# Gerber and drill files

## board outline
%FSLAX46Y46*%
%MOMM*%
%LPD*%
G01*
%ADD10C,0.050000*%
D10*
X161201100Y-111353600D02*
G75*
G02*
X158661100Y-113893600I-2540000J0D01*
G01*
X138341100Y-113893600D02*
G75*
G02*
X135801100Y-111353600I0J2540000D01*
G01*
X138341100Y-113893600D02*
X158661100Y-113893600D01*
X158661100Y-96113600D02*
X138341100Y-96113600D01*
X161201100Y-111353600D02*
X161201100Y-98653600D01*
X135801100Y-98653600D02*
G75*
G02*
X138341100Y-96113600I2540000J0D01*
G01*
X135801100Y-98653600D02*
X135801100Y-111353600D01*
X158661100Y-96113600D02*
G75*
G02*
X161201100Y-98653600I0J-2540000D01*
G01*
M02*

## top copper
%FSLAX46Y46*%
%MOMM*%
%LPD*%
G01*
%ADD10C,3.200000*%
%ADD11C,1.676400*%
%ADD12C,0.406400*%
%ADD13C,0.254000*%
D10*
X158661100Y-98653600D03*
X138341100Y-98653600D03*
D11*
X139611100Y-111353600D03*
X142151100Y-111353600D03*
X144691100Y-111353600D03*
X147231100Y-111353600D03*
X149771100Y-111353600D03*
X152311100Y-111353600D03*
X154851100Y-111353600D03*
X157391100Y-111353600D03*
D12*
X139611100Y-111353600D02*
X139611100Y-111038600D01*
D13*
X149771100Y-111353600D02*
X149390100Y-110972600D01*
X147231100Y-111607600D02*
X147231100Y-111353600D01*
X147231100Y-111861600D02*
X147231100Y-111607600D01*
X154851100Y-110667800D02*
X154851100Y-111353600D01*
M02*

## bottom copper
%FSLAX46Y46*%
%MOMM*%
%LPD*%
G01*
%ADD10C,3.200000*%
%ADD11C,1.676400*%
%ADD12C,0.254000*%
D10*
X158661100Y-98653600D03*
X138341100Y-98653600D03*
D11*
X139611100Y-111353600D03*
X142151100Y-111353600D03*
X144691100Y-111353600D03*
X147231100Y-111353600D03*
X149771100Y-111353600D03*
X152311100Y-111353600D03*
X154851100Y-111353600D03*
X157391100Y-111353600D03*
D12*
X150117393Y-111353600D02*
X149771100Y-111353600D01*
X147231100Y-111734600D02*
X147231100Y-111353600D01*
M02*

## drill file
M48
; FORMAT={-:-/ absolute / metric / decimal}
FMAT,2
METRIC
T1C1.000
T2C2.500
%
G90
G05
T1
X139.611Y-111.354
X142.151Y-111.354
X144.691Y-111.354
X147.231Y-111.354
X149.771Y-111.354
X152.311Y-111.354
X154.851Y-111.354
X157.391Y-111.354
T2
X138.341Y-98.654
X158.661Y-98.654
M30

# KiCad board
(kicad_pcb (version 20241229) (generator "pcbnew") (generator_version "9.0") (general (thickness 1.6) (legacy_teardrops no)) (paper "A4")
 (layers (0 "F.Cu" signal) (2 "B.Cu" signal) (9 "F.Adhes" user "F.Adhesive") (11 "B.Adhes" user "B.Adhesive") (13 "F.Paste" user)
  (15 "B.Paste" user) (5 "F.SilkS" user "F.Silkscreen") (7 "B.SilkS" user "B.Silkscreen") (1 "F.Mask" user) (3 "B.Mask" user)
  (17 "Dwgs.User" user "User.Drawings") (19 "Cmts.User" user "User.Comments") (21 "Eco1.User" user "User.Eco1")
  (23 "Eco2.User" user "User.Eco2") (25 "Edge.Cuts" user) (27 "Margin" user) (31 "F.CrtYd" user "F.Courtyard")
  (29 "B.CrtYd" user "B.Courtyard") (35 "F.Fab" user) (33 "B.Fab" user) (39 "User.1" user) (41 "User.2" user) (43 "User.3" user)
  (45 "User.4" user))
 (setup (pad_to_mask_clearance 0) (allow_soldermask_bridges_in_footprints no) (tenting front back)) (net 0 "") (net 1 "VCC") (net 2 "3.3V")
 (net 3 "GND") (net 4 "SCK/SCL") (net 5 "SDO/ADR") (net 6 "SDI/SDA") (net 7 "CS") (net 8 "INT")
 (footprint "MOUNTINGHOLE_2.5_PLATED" (layer "F.Cu") (at 158.6611 98.6536)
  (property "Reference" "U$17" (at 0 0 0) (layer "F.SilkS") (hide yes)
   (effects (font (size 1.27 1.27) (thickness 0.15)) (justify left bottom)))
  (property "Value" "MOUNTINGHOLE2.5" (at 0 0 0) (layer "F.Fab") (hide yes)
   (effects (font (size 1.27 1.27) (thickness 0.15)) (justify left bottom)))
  (pad "P$1" thru_hole circle (at 0 0) (size 3.2 3.2) (drill 2.5) (layers "*.Cu" "*.Mask") (remove_unused_layers no)
   (solder_mask_margin 0.0508) (thermal_bridge_angle 0))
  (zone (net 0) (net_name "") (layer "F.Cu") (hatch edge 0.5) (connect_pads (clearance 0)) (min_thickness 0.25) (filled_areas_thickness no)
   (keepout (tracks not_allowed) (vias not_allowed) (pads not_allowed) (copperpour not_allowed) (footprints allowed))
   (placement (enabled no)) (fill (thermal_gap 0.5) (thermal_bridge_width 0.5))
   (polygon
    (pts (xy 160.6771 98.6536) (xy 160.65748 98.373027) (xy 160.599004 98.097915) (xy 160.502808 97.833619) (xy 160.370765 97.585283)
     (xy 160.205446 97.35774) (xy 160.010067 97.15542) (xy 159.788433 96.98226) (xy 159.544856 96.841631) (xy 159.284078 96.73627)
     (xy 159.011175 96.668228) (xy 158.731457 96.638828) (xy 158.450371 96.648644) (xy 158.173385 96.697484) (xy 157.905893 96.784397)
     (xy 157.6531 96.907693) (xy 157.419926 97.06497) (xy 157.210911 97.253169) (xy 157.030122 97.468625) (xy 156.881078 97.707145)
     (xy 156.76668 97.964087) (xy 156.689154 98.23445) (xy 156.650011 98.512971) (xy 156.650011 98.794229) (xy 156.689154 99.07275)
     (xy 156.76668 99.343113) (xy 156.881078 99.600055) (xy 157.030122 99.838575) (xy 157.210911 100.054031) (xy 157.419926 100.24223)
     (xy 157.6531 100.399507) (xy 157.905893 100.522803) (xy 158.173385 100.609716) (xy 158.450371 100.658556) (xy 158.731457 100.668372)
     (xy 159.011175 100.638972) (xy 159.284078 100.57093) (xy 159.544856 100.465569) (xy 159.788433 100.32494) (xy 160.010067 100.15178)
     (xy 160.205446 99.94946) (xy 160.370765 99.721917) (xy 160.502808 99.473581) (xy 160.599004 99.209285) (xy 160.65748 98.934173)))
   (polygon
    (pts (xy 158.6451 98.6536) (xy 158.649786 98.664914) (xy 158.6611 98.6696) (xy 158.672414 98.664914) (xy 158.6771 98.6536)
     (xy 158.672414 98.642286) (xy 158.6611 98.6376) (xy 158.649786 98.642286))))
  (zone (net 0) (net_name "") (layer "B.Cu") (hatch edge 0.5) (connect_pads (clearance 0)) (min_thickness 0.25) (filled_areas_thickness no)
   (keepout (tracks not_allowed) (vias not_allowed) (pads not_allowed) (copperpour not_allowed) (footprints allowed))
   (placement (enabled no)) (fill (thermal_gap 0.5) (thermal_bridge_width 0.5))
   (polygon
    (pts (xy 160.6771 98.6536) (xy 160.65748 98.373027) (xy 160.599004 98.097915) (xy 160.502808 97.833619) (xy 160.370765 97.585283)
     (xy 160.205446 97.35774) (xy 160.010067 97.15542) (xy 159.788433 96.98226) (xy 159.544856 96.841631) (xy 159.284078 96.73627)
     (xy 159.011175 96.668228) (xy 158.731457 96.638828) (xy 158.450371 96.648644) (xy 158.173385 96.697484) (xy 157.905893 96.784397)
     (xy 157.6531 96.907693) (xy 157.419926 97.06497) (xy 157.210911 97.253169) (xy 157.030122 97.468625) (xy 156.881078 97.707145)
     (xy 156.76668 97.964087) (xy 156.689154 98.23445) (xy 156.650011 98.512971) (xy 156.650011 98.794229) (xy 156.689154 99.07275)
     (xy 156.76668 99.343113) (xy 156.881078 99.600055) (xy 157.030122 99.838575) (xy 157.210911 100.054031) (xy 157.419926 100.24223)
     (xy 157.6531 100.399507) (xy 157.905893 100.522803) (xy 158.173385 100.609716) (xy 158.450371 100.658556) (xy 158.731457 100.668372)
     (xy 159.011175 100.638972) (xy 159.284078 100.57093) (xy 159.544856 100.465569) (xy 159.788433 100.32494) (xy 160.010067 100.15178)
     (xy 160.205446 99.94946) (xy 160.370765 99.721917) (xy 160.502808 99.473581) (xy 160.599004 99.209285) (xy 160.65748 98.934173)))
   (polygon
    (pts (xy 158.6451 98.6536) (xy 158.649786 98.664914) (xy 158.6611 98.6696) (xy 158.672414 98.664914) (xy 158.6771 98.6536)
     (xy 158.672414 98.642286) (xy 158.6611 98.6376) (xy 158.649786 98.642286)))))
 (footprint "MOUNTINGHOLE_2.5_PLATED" (layer "F.Cu") (at 138.3411 98.6536)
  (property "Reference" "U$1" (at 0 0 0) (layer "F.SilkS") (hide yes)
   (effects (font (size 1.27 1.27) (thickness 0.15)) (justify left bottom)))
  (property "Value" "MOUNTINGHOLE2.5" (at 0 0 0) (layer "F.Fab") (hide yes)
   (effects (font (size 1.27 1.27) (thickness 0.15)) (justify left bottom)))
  (pad "P$1" thru_hole circle (at 0 0) (size 3.2 3.2) (drill 2.5) (layers "*.Cu" "*.Mask") (remove_unused_layers no)
   (solder_mask_margin 0.0508) (thermal_bridge_angle 0))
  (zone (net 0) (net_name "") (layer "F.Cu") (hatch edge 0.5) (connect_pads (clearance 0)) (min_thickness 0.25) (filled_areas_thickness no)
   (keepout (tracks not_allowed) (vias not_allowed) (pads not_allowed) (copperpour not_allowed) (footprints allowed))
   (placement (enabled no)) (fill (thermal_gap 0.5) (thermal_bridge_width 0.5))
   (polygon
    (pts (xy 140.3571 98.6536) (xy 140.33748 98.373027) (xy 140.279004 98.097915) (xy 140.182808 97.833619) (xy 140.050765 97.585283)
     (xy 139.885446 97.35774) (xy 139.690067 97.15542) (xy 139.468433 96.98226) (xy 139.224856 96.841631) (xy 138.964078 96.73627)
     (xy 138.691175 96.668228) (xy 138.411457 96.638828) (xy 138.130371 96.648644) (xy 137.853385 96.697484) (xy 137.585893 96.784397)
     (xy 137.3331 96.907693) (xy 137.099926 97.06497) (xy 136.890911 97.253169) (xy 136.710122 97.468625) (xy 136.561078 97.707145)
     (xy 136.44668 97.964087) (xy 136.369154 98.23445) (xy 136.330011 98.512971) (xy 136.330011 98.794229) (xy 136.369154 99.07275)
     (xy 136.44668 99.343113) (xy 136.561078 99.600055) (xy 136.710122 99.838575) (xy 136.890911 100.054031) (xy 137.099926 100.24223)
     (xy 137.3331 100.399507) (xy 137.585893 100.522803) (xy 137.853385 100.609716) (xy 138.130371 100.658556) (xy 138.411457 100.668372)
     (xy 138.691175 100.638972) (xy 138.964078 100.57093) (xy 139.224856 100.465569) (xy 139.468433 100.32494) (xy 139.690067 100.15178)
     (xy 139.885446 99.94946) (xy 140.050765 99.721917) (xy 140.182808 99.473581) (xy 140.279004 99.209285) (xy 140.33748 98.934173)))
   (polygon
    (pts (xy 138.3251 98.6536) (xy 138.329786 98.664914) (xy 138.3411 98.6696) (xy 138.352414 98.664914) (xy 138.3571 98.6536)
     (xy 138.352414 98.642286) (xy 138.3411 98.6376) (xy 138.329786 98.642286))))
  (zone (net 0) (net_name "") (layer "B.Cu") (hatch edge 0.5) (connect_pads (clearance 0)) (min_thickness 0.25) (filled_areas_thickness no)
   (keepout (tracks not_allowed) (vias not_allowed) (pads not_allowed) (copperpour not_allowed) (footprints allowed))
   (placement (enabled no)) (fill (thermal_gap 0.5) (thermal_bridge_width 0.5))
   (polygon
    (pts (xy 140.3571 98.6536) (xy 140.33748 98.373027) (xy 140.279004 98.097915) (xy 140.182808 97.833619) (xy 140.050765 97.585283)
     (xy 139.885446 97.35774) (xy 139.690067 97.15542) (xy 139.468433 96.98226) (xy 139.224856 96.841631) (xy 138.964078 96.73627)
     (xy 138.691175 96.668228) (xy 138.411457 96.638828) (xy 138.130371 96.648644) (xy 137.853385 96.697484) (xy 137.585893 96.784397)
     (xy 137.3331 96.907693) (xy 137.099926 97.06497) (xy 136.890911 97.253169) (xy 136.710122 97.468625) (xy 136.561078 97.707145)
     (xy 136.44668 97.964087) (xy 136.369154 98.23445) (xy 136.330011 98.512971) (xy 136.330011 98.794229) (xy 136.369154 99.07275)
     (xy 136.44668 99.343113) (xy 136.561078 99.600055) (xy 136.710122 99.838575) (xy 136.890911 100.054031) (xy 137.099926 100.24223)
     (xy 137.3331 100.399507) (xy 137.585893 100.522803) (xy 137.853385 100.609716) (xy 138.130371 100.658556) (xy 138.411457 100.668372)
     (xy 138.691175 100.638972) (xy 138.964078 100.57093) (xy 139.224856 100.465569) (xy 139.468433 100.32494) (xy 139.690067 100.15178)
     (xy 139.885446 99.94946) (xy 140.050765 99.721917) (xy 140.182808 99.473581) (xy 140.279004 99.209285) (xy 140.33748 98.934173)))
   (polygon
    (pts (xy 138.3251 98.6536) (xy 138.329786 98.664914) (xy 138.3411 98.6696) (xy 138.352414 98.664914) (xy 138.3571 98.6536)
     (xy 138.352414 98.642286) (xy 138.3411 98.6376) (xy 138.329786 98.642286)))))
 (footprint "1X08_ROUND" (layer "F.Cu") (at 148.5011 111.3536)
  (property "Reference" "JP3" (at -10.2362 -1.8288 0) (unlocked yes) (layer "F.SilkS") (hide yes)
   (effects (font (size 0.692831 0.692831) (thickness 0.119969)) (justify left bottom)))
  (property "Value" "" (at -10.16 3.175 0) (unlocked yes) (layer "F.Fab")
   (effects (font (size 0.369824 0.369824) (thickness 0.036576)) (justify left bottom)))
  (pad "1" thru_hole circle (at -8.89 0 90) (size 1.6764 1.6764) (drill 1) (layers "*.Cu" "*.Mask") (remove_unused_layers no) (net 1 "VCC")
   (solder_mask_margin 0.0508) (thermal_bridge_angle 0))
  (pad "2" thru_hole circle (at -6.35 0 90) (size 1.6764 1.6764) (drill 1) (layers "*.Cu" "*.Mask") (remove_unused_layers no) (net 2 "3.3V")
   (solder_mask_margin 0.0508) (thermal_bridge_angle 0))
  (pad "3" thru_hole circle (at -3.81 0 90) (size 1.6764 1.6764) (drill 1) (layers "*.Cu" "*.Mask") (remove_unused_layers no) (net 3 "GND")
   (solder_mask_margin 0.0508) (thermal_bridge_angle 0))
  (pad "4" thru_hole circle (at -1.27 0 90) (size 1.6764 1.6764) (drill 1) (layers "*.Cu" "*.Mask") (remove_unused_layers no)
   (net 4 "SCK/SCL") (solder_mask_margin 0.0508) (thermal_bridge_angle 0))
  (pad "5" thru_hole circle (at 1.27 0 90) (size 1.6764 1.6764) (drill 1) (layers "*.Cu" "*.Mask") (remove_unused_layers no)
   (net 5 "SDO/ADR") (solder_mask_margin 0.0508) (thermal_bridge_angle 0))
  (pad "6" thru_hole circle (at 3.81 0 90) (size 1.6764 1.6764) (drill 1) (layers "*.Cu" "*.Mask") (remove_unused_layers no)
   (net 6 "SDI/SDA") (solder_mask_margin 0.0508) (thermal_bridge_angle 0))
  (pad "7" thru_hole circle (at 6.35 0 90) (size 1.6764 1.6764) (drill 1) (layers "*.Cu" "*.Mask") (remove_unused_layers no) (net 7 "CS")
   (solder_mask_margin 0.0508) (thermal_bridge_angle 0))
  (pad "8" thru_hole circle (at 8.89 0 90) (size 1.6764 1.6764) (drill 1) (layers "*.Cu" "*.Mask") (remove_unused_layers no) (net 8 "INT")
   (solder_mask_margin 0.0508) (thermal_bridge_angle 0)))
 (gr_arc (start 161.2011 111.3536) (mid 160.457151 113.149651) (end 158.6611 113.8936) (stroke (width 0.05) (type solid))
  (layer "Edge.Cuts"))
 (gr_arc (start 138.3411 113.8936) (mid 136.545049 113.149651) (end 135.8011 111.3536) (stroke (width 0.05) (type solid))
  (layer "Edge.Cuts"))
 (gr_line (start 138.3411 113.8936) (end 158.6611 113.8936) (stroke (width 0.05) (type solid)) (layer "Edge.Cuts"))
 (gr_line (start 158.6611 96.1136) (end 138.3411 96.1136) (stroke (width 0.05) (type solid)) (layer "Edge.Cuts"))
 (gr_line (start 161.2011 111.3536) (end 161.2011 98.6536) (stroke (width 0.05) (type solid)) (layer "Edge.Cuts"))
 (gr_arc (start 135.8011 98.6536) (mid 136.545049 96.857549) (end 138.3411 96.1136) (stroke (width 0.05) (type solid)) (layer "Edge.Cuts"))
 (gr_line (start 135.8011 98.6536) (end 135.8011 111.3536) (stroke (width 0.05) (type solid)) (layer "Edge.Cuts"))
 (gr_arc (start 158.6611 96.1136) (mid 160.457151 96.857549) (end 161.2011 98.6536) (stroke (width 0.05) (type solid)) (layer "Edge.Cuts"))
 (segment (start 139.6111 111.3536) (end 139.6111 111.0386) (width 0.4064) (layer "F.Cu") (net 1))
 (segment (start 149.7711 111.3536) (end 149.3901 110.9726) (width 0.254) (layer "F.Cu") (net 5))
 (segment (start 150.117393 111.3536) (end 149.7711 111.3536) (width 0.254) (layer "B.Cu") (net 5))
 (segment (start 147.2311 111.6076) (end 147.2311 111.3536) (width 0.254) (layer "F.Cu") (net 4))
 (segment (start 147.2311 111.8616) (end 147.2311 111.6076) (width 0.254) (layer "F.Cu") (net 4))
 (segment (start 147.2311 111.7346) (end 147.2311 111.3536) (width 0.254) (layer "B.Cu") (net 4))
 (segment (start 154.8511 110.6678) (end 154.8511 111.3536) (width 0.254) (layer "F.Cu") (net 7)))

